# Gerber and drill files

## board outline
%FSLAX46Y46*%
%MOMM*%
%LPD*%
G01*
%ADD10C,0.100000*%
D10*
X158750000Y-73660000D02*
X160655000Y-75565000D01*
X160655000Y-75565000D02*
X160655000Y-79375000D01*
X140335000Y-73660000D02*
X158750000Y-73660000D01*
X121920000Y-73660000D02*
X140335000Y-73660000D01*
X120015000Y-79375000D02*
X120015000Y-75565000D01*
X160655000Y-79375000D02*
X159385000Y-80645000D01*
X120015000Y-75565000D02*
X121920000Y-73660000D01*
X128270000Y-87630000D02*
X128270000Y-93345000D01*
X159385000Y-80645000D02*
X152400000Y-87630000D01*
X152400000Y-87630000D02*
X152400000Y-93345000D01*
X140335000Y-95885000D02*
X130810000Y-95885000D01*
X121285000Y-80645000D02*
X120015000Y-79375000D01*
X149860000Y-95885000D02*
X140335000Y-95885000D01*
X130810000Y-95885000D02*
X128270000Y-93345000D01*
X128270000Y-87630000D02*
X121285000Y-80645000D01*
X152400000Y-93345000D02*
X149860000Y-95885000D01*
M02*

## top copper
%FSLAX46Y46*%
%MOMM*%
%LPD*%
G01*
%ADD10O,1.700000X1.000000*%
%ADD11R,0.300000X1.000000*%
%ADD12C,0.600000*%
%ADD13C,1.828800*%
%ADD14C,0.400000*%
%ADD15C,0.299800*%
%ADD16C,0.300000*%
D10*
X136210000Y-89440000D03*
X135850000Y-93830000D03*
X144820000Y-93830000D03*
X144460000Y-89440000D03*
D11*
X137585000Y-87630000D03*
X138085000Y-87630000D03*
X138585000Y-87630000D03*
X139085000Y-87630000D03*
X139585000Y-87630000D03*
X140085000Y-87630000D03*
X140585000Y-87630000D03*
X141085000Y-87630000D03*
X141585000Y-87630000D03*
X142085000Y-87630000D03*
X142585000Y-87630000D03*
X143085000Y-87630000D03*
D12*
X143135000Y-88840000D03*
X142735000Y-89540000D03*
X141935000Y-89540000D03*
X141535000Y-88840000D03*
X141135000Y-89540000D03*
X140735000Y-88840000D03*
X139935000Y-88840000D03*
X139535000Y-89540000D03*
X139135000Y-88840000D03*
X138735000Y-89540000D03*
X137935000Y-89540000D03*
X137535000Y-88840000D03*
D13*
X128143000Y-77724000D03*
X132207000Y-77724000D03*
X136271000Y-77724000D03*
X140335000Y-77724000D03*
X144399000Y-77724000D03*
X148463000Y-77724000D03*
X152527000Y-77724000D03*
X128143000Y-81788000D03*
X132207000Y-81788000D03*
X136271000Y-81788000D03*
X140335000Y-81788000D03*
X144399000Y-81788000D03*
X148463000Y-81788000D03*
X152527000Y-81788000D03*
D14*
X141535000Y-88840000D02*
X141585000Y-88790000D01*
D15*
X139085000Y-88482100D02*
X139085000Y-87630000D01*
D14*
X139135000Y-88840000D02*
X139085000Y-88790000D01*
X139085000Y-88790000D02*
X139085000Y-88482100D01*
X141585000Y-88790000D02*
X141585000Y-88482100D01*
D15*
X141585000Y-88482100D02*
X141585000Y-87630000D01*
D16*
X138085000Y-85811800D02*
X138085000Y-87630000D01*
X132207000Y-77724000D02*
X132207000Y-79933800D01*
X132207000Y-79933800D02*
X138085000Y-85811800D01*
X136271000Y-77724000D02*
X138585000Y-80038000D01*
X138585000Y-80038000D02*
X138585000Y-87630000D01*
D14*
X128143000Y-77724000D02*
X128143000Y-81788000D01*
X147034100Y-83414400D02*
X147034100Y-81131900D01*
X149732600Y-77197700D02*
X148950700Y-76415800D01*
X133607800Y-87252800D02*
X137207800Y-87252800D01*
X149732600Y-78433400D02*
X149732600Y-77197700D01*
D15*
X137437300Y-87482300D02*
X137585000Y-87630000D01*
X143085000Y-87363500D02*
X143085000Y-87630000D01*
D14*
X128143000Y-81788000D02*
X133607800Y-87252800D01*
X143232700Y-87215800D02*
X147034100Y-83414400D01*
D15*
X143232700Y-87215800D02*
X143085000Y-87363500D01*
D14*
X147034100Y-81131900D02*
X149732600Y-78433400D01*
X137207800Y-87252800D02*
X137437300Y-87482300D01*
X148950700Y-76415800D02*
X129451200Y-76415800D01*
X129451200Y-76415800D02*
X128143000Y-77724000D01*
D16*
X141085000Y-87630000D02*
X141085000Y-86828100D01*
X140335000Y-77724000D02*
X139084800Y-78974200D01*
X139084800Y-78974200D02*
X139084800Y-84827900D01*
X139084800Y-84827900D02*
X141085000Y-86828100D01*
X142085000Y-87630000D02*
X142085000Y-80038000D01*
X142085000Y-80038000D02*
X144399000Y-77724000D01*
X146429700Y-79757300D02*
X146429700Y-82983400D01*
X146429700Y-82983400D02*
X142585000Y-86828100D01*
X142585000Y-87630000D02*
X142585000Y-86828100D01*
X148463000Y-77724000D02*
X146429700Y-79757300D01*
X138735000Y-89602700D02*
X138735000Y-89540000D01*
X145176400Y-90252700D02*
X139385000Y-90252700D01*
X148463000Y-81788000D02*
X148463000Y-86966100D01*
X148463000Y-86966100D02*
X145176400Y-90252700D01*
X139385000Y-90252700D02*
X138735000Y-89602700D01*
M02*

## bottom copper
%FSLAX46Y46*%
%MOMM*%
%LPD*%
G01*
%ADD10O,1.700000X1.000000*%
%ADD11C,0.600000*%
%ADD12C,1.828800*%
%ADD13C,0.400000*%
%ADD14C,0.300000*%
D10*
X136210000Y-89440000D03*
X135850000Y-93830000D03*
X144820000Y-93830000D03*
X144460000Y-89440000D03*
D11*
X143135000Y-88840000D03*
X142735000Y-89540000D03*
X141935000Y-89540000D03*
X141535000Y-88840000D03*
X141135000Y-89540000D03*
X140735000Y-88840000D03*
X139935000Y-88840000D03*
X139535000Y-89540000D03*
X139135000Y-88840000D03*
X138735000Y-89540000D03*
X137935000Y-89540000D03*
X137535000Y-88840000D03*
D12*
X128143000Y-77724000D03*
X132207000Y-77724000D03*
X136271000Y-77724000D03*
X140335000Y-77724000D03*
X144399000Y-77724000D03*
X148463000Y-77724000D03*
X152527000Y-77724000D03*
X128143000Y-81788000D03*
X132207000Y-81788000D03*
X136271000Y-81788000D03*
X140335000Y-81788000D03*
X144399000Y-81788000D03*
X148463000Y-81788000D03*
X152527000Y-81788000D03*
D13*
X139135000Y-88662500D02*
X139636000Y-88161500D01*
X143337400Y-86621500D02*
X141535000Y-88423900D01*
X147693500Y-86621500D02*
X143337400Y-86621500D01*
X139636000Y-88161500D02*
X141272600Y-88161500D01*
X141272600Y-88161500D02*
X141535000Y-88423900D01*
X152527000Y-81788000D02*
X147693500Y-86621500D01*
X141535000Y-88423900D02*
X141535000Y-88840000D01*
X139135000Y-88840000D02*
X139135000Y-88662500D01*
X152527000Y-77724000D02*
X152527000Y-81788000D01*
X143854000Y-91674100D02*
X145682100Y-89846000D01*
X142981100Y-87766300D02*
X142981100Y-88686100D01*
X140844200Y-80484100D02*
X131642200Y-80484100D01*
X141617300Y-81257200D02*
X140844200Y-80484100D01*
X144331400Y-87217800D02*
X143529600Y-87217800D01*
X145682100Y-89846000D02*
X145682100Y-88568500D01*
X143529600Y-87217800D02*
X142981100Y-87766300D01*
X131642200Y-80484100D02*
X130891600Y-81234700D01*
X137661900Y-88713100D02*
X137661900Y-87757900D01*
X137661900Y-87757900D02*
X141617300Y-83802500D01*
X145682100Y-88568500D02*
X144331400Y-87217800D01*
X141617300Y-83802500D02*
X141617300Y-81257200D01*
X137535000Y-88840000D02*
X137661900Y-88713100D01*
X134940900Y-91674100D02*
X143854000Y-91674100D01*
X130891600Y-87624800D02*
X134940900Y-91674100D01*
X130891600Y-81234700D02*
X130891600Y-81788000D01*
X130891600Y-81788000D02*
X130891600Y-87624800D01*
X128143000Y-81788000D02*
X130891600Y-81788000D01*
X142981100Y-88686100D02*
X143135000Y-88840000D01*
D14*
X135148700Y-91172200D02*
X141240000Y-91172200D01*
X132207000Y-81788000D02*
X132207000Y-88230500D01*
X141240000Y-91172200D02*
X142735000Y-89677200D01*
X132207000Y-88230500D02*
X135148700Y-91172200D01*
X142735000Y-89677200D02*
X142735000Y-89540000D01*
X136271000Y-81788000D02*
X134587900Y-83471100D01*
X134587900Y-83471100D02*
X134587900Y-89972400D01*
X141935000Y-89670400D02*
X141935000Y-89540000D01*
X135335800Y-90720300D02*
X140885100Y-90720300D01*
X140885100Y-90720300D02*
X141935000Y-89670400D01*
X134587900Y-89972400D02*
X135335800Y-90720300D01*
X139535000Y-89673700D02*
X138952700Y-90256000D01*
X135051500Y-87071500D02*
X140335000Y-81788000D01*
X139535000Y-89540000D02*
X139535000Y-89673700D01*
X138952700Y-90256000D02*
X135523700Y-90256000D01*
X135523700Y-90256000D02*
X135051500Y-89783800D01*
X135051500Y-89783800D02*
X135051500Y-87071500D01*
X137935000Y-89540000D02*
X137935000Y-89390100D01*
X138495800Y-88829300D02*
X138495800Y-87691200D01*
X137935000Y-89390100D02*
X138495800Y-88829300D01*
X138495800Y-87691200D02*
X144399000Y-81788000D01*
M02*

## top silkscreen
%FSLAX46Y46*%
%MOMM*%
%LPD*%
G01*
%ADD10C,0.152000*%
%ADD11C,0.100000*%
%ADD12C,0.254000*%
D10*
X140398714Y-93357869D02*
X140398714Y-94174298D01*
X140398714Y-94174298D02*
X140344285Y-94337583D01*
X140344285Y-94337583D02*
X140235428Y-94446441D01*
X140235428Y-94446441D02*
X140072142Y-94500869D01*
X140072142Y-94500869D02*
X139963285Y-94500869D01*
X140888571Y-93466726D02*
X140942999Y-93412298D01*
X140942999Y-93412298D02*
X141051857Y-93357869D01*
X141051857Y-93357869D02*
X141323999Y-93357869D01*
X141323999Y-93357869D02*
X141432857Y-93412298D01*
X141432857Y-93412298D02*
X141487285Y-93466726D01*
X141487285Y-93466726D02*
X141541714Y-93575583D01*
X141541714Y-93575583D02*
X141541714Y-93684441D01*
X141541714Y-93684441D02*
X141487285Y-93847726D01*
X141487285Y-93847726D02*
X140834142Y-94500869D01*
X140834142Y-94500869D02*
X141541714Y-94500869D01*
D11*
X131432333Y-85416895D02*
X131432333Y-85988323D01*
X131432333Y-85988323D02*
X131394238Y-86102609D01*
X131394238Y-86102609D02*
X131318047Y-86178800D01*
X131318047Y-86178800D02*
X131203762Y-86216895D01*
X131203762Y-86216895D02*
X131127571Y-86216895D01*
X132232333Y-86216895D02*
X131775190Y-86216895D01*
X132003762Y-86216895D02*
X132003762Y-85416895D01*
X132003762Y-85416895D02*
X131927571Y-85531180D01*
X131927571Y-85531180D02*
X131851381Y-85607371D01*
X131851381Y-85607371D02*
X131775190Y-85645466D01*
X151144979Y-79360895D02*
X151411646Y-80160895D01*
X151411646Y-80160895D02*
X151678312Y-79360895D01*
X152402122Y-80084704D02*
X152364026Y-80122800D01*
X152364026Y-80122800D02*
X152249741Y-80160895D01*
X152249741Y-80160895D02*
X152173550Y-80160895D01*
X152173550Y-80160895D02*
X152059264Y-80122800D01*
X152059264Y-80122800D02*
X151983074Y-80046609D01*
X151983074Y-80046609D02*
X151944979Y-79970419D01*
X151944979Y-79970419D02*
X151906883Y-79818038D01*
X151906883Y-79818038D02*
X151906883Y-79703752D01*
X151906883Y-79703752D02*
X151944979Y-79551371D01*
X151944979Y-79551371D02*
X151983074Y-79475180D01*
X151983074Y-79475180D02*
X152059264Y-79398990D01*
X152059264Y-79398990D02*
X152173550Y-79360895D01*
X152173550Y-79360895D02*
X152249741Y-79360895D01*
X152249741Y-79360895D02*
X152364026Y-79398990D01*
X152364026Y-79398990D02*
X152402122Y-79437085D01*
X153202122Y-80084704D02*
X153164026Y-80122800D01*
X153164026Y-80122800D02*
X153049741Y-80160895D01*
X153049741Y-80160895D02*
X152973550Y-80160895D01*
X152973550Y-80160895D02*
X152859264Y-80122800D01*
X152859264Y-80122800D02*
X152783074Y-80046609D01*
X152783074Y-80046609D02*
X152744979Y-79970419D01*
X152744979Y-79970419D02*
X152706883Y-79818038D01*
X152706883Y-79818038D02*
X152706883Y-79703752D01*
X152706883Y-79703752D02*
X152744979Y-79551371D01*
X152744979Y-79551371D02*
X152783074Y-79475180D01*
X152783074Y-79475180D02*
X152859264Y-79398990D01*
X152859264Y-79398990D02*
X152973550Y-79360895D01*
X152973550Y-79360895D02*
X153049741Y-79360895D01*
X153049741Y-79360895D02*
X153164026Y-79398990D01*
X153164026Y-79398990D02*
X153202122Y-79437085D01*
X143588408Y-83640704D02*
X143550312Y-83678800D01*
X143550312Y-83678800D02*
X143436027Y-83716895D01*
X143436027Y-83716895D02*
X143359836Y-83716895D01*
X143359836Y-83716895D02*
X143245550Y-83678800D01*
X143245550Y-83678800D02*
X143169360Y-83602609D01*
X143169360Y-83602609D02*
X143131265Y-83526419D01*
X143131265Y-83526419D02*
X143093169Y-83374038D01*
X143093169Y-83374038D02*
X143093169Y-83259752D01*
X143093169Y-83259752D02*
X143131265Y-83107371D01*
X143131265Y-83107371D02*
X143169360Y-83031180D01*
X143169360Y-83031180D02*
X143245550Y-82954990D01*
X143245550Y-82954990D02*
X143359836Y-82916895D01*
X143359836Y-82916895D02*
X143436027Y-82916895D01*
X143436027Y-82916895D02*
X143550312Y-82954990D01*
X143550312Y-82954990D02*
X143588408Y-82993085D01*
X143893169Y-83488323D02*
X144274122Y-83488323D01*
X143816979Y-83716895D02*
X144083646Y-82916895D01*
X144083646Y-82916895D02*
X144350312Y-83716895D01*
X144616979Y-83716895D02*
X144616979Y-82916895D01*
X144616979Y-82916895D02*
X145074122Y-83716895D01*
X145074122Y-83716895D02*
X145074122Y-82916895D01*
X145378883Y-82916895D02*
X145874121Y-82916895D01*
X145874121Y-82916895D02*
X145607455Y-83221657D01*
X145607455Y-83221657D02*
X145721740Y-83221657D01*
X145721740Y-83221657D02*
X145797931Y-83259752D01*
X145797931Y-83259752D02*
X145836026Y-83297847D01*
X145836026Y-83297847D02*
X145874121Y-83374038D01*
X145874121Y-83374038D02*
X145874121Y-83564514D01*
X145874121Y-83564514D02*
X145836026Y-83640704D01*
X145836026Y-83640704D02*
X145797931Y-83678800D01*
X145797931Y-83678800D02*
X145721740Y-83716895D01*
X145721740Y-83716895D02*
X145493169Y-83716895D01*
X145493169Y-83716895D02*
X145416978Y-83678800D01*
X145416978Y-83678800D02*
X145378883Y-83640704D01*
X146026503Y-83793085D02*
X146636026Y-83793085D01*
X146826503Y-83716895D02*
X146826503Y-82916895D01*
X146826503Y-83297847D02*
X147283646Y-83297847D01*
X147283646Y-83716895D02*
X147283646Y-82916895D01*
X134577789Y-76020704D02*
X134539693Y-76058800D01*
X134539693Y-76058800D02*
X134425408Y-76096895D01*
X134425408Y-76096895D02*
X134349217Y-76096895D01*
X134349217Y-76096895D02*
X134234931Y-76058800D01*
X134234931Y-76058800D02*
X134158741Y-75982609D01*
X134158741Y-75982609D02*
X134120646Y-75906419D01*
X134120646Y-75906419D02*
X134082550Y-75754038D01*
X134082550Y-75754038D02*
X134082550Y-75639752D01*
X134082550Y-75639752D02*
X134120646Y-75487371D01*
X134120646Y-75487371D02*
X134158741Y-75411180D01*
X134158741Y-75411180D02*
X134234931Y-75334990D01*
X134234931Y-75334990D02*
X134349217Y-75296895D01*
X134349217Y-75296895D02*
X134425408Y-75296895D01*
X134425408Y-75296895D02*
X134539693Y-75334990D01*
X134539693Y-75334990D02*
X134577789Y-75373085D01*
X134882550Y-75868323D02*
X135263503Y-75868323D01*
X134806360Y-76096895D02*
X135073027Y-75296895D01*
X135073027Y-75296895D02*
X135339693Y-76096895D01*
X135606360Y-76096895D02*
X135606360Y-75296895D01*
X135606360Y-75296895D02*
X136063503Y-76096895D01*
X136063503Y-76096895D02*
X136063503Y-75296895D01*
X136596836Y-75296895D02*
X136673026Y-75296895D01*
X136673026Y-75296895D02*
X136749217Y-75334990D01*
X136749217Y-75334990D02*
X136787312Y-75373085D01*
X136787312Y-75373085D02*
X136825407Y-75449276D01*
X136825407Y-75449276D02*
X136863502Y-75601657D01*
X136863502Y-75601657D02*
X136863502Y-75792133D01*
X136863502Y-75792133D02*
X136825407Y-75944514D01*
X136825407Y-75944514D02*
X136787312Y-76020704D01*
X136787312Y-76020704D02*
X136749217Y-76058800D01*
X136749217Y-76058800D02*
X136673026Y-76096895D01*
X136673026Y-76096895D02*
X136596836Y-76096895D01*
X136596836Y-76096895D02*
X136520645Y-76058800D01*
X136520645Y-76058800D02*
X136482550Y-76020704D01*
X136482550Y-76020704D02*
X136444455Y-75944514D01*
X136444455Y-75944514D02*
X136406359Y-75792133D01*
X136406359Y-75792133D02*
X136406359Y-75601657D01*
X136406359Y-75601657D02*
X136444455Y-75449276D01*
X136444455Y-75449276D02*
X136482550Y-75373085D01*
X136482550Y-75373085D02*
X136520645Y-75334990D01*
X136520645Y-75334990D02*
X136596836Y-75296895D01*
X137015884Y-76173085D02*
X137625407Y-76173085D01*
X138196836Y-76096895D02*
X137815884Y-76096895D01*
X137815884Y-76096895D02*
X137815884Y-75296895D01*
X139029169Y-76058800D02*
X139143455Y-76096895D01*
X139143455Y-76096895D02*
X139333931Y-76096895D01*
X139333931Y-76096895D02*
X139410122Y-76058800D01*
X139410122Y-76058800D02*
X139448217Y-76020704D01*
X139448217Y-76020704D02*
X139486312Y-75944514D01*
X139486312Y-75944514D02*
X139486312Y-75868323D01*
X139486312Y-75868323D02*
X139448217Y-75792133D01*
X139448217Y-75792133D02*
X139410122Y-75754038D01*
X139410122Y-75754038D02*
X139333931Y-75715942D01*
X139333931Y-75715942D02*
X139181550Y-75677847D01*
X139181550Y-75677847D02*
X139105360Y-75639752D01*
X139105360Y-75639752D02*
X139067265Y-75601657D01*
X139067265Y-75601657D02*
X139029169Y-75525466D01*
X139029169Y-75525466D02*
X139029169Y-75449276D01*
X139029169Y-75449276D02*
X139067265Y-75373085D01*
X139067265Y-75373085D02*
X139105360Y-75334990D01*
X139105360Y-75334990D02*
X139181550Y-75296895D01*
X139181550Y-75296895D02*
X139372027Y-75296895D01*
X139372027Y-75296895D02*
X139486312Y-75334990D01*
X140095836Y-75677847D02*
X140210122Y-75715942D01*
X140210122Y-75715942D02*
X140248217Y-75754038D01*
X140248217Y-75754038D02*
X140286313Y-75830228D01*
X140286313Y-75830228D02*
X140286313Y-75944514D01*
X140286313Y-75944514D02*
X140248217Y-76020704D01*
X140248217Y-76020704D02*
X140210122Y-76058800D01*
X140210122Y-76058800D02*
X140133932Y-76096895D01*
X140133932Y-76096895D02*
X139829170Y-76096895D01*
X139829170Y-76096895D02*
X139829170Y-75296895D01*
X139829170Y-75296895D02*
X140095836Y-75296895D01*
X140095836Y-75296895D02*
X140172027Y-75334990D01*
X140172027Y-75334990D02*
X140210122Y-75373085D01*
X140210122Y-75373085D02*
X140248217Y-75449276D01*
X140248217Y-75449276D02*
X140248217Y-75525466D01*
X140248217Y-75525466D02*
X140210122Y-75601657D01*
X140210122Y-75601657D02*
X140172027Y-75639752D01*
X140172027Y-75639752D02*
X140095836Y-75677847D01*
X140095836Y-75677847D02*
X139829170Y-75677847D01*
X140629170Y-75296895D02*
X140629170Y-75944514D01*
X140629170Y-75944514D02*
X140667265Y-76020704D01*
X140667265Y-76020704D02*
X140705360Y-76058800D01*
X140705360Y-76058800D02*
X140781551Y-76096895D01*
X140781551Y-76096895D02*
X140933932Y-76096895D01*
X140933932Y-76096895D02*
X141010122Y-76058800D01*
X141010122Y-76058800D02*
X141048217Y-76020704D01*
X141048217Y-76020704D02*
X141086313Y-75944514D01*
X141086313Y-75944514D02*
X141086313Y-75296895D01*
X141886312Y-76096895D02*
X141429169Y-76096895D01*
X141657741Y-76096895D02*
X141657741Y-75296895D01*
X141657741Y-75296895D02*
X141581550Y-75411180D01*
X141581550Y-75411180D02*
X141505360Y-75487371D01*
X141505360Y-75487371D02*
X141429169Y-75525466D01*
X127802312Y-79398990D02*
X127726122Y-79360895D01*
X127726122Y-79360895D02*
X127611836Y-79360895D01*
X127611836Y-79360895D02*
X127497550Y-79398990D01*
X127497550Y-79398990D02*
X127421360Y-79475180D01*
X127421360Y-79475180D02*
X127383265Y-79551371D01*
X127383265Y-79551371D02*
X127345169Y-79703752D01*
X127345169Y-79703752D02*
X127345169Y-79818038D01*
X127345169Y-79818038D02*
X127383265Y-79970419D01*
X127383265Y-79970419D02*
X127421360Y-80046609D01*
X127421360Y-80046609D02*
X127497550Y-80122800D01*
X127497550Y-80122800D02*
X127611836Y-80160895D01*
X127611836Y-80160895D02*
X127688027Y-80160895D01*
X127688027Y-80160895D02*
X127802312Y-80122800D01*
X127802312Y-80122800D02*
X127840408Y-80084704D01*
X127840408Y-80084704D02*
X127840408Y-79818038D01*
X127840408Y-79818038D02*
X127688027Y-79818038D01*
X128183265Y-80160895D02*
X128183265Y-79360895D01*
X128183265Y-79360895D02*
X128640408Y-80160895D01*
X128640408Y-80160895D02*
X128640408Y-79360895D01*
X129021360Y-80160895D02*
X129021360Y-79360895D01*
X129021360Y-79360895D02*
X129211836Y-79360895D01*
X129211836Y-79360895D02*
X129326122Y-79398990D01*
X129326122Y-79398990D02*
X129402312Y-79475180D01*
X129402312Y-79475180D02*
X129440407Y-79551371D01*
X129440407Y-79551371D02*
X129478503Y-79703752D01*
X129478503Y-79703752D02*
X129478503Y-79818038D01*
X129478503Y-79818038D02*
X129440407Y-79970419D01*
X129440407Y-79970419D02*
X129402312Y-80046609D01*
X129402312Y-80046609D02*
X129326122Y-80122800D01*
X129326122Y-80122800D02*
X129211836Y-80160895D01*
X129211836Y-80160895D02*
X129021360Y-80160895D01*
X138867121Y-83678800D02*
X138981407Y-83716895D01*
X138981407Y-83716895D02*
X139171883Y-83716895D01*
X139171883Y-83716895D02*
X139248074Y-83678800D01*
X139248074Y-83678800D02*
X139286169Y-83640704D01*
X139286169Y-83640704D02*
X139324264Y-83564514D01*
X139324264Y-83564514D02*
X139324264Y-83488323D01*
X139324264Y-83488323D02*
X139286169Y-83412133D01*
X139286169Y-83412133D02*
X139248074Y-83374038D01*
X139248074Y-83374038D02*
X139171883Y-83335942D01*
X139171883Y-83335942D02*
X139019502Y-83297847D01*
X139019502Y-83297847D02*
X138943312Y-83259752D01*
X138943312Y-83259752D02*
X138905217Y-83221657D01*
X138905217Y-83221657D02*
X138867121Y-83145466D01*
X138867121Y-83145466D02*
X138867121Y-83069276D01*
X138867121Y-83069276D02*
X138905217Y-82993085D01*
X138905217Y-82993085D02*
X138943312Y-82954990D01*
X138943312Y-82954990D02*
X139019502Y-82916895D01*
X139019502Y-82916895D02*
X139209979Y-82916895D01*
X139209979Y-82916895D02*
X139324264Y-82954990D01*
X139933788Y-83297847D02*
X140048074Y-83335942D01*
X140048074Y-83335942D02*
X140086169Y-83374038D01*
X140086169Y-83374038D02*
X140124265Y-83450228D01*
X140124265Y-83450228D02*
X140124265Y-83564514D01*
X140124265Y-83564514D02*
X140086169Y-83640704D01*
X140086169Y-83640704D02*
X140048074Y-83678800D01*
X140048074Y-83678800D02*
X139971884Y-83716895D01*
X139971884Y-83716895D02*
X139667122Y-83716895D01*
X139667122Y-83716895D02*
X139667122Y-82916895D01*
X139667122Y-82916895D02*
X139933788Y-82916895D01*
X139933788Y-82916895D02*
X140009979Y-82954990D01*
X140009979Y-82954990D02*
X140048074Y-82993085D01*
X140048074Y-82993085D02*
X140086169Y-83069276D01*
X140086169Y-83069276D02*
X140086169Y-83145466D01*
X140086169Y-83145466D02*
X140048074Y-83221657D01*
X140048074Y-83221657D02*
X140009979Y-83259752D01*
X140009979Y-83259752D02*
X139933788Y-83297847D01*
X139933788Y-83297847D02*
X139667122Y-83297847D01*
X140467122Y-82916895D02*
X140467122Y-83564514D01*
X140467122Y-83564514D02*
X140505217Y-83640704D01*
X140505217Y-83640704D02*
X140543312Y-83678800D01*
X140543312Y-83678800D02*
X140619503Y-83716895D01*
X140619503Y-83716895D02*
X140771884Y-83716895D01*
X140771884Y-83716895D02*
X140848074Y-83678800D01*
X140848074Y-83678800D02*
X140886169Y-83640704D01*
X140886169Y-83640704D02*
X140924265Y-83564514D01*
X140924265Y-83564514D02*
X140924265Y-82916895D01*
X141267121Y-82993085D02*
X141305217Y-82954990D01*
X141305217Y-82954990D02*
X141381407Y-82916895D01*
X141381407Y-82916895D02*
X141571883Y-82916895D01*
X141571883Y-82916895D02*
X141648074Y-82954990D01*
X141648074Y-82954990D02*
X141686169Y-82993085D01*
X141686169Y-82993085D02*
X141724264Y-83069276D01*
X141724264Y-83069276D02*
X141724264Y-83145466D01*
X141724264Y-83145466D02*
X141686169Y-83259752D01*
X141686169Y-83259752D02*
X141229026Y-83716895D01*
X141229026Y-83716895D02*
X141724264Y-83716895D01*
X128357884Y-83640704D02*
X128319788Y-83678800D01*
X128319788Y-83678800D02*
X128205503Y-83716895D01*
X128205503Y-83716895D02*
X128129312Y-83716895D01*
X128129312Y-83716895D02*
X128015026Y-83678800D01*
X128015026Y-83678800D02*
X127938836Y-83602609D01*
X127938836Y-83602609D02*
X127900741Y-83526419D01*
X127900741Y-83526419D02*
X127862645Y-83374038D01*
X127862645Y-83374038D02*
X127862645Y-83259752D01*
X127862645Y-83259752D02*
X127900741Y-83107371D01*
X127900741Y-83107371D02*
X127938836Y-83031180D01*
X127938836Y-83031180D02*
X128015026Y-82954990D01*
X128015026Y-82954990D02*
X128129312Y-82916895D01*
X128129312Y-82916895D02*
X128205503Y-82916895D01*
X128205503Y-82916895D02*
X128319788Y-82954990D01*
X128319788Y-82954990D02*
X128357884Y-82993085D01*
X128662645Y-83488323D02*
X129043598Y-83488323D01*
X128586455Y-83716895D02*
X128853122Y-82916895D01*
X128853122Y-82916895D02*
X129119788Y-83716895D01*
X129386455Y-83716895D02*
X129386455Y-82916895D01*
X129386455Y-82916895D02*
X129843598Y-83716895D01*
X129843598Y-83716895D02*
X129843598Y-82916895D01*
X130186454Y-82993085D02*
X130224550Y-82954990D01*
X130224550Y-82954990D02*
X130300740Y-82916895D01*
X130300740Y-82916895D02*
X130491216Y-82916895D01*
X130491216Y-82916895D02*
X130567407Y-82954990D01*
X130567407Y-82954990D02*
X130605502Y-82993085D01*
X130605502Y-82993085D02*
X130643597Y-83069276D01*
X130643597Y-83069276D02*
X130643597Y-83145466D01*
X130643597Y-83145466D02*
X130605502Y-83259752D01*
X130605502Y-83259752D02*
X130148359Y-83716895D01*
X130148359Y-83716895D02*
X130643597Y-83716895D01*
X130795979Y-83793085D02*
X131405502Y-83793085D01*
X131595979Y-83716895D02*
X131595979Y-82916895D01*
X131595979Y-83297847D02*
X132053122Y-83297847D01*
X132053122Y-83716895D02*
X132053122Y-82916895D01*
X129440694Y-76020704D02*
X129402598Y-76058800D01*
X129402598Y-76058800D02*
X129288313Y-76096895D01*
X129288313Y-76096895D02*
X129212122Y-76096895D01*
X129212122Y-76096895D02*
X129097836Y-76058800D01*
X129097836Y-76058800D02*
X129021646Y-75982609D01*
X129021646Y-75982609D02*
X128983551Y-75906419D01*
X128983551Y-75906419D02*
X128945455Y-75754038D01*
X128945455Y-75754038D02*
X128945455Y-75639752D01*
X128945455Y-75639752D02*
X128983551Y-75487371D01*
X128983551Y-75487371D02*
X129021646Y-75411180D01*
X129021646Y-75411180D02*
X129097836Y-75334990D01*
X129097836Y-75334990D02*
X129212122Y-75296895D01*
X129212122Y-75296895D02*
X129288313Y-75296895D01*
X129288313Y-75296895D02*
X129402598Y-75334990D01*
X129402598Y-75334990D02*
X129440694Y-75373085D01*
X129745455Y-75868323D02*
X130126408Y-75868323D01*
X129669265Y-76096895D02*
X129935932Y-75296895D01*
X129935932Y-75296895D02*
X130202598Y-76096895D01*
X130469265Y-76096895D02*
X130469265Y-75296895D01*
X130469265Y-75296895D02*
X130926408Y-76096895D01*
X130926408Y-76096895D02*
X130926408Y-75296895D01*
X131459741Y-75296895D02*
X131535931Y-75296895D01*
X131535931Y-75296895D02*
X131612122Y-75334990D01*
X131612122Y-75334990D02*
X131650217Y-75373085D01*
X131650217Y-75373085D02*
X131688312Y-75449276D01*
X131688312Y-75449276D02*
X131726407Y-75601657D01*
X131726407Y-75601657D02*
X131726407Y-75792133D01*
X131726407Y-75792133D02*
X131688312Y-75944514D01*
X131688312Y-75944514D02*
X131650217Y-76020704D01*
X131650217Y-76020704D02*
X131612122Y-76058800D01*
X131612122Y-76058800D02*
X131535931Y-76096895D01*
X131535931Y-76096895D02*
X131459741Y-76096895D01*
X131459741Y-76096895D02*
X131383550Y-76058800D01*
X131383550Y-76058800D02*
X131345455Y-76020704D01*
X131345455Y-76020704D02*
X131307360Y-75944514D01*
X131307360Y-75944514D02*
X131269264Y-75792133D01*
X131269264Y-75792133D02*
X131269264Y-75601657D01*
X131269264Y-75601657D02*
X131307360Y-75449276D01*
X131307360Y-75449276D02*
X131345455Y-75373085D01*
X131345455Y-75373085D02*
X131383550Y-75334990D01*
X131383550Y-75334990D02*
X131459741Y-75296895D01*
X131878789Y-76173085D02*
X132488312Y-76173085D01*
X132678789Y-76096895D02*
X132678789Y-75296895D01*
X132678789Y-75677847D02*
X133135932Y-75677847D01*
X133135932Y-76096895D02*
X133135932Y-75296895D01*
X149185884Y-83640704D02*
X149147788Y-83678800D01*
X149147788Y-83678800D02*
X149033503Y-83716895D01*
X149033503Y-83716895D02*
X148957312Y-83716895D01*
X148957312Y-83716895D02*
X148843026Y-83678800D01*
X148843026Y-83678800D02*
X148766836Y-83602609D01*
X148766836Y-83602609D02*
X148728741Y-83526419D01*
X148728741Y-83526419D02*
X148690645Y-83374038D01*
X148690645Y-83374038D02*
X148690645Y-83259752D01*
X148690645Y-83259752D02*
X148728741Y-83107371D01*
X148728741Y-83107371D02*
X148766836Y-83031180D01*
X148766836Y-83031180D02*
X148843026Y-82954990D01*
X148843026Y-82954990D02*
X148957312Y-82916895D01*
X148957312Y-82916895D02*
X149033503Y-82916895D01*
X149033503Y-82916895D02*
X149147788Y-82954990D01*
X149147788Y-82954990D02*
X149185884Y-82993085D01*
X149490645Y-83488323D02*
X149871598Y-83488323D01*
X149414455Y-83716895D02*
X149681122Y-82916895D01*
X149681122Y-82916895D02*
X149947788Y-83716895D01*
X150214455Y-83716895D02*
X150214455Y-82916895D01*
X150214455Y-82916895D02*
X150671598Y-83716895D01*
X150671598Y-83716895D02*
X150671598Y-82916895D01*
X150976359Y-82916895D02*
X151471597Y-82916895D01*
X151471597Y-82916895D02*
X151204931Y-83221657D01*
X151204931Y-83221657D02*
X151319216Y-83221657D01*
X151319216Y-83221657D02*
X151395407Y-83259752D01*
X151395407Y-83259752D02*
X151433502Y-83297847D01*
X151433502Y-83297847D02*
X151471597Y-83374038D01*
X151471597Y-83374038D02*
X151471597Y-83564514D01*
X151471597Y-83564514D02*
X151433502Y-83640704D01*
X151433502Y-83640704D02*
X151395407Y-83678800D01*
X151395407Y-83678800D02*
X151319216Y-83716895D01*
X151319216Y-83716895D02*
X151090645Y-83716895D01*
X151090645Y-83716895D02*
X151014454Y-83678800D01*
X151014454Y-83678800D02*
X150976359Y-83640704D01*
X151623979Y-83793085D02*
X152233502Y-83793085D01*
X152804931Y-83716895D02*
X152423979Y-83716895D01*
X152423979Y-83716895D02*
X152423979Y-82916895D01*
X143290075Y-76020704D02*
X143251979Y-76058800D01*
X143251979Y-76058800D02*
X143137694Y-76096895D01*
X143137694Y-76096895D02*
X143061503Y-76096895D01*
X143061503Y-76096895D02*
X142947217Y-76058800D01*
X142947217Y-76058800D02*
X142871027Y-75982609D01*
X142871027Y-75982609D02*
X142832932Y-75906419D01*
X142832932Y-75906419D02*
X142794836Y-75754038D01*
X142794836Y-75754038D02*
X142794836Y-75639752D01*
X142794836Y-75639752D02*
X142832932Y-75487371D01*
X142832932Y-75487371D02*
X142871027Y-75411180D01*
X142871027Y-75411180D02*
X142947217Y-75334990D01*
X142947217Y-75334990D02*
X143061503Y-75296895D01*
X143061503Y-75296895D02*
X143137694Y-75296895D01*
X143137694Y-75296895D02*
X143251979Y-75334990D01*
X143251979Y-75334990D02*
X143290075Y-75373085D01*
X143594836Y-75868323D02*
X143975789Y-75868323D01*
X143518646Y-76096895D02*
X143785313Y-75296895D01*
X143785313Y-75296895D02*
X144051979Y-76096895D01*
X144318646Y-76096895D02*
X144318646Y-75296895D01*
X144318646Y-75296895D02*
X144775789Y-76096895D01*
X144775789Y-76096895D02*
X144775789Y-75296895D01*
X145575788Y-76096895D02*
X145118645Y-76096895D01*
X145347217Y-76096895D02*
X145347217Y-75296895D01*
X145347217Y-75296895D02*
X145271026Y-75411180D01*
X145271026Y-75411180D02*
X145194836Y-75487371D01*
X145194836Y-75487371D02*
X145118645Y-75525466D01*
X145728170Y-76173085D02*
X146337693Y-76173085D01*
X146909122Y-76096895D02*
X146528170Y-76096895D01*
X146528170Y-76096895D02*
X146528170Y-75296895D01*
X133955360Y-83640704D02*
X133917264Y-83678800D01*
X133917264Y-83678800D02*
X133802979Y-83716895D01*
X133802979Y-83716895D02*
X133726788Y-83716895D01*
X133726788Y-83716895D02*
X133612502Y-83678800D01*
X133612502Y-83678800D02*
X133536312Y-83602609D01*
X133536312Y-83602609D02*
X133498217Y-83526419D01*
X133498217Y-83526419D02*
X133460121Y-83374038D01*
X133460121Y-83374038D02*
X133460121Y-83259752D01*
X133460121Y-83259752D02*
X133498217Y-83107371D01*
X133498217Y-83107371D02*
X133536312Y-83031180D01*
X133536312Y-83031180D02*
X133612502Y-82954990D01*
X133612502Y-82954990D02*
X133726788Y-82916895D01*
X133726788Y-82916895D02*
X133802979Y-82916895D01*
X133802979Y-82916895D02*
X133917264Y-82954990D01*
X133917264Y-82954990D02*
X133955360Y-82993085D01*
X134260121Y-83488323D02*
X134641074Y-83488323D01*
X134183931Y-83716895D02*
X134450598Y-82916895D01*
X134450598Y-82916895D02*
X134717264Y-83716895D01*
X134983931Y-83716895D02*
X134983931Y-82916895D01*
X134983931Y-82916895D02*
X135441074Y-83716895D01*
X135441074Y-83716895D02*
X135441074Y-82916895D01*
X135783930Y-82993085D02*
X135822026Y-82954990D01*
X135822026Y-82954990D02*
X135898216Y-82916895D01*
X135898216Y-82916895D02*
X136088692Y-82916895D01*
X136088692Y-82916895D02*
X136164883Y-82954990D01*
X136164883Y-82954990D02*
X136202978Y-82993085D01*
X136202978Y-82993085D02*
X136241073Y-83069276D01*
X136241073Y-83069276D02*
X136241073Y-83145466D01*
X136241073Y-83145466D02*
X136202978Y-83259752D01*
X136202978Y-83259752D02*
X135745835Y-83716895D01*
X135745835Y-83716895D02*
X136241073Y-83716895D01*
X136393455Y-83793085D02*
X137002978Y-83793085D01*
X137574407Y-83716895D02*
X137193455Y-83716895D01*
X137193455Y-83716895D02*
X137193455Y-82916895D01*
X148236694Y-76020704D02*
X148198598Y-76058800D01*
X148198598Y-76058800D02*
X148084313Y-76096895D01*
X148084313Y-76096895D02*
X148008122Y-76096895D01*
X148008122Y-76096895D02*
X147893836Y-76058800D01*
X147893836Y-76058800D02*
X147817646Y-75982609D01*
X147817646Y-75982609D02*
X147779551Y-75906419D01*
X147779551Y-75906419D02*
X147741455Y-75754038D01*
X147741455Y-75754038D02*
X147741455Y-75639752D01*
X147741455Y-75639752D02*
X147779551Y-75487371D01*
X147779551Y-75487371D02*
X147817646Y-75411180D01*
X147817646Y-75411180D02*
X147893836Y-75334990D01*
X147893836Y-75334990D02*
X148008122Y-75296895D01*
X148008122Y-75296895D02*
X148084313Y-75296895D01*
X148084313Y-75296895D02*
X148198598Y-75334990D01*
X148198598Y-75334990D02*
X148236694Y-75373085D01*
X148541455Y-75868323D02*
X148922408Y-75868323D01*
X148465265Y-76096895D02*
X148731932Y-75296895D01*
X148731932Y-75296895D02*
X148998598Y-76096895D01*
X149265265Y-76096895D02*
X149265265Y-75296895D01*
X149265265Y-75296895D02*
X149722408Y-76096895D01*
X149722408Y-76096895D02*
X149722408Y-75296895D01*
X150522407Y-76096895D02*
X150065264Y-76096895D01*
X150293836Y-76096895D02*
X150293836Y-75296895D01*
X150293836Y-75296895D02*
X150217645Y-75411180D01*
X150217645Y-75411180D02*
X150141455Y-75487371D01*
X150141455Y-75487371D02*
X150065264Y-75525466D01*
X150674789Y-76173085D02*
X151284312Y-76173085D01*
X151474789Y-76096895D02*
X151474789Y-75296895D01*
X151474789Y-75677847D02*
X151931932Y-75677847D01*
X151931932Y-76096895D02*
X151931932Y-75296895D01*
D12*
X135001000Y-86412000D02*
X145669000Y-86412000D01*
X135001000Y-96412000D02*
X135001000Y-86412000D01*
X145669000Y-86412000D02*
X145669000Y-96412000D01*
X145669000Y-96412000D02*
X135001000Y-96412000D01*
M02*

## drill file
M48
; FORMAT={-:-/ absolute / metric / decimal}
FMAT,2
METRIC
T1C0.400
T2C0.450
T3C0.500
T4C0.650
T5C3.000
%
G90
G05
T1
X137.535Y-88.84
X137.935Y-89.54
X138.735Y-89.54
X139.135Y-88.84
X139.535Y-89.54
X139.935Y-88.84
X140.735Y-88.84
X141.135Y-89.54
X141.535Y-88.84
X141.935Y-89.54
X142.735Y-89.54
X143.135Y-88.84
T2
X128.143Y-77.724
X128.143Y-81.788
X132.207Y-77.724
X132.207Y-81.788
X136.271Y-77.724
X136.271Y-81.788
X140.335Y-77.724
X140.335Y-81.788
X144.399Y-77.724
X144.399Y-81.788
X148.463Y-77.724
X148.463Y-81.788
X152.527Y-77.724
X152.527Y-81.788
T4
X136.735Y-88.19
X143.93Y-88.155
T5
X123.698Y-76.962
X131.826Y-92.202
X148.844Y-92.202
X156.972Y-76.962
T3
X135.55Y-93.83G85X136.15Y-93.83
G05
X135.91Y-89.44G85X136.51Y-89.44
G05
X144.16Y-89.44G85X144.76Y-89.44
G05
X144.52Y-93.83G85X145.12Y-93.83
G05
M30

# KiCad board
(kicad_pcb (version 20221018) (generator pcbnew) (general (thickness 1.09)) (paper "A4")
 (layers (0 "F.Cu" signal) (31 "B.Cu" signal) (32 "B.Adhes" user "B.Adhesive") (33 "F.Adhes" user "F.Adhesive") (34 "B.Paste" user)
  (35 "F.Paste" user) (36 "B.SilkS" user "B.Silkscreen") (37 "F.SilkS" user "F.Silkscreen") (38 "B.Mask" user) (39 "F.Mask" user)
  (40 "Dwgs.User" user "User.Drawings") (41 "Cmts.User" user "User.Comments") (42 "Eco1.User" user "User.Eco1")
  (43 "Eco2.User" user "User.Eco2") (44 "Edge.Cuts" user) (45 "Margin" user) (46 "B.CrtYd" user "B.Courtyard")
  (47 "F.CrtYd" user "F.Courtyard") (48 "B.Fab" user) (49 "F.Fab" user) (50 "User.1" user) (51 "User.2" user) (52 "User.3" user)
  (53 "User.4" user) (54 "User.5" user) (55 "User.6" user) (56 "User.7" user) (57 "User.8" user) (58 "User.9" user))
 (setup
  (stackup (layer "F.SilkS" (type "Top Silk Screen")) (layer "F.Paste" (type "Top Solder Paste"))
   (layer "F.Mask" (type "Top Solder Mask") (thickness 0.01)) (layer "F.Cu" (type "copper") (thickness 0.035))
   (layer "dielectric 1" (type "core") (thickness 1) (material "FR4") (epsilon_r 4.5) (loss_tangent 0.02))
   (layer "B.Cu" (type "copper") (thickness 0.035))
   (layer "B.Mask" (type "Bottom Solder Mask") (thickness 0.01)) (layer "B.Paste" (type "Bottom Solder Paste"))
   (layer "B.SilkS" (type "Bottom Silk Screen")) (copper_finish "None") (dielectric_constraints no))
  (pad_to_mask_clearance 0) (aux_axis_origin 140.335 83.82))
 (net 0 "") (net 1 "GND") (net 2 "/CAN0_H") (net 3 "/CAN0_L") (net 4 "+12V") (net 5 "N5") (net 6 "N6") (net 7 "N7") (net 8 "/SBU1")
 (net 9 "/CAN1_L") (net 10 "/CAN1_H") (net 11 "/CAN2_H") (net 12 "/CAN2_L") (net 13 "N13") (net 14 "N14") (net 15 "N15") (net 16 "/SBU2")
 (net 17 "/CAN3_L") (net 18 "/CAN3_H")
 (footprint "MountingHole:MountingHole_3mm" (layer "F.Cu") (at 123.698 76.962)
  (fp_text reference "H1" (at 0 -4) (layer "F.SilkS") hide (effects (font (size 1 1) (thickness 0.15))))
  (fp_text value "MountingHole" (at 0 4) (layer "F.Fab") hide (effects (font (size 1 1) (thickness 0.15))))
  (pad "" np_thru_hole circle (at 0 0) (size 3 3) (drill 3) (layers "*.Cu" "*.Mask")))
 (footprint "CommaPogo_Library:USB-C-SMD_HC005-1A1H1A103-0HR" (layer "F.Cu") (at 140.335 90.73)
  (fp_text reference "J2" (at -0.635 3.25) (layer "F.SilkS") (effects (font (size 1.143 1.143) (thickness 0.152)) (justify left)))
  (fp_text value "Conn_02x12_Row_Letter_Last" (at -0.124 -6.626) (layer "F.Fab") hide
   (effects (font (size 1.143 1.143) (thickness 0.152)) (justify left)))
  (fp_line (start -5.334 -4.318) (end 5.334 -4.318) (stroke (width 0.254) (type solid)) (layer "F.SilkS"))
  (fp_line (start -5.334 5.682) (end -5.334 -4.318) (stroke (width 0.254) (type solid)) (layer "F.SilkS"))
  (fp_line (start 5.334 -4.318) (end 5.334 5.682) (stroke (width 0.254) (type solid)) (layer "F.SilkS"))
  (fp_line (start 5.334 5.682) (end -5.334 5.682) (stroke (width 0.254) (type solid)) (layer "F.SilkS"))
  (pad "" np_thru_hole circle (at -3.6 -2.54) (size 0.65 0.65) (drill 0.65) (layers "*.Cu" "*.Mask"))
  (pad "" np_thru_hole circle (at 3.595 -2.575) (size 0.65 0.65) (drill 0.65) (layers "*.Cu" "*.Mask"))
  (pad "1" thru_hole oval (at -4.125 -1.29 90) (size 1 1.7) (drill oval 0.5 1.1) (layers "*.Cu" "*.Paste" "*.Mask"))
  (pad "2" thru_hole oval (at -4.485 3.1 90) (size 1 1.7) (drill oval 0.5 1.1) (layers "*.Cu" "*.Paste" "*.Mask"))
  (pad "3" thru_hole oval (at 4.485 3.1 90) (size 1 1.7) (drill oval 0.5 1.1) (layers "*.Cu" "*.Paste" "*.Mask"))
  (pad "4" thru_hole oval (at 4.125 -1.29 90) (size 1 1.7) (drill oval 0.5 1.1) (layers "*.Cu" "*.Paste" "*.Mask"))
  (pad "A1" smd rect (at -2.75 -3.1) (size 0.3 1) (layers "F.Cu" "F.Paste" "F.Mask") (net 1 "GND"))
  (pad "A2" smd rect (at -2.25 -3.1) (size 0.3 1) (layers "F.Cu" "F.Paste" "F.Mask") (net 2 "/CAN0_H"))
  (pad "A3" smd rect (at -1.75 -3.1) (size 0.3 1) (layers "F.Cu" "F.Paste" "F.Mask") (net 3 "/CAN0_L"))
  (pad "A4" smd rect (at -1.25 -3.1) (size 0.3 1) (layers "F.Cu" "F.Paste" "F.Mask") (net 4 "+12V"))
  (pad "A5" smd rect (at -0.75 -3.1) (size 0.3 1) (layers "F.Cu" "F.Paste" "F.Mask") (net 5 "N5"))
  (pad "A6" smd rect (at -0.25 -3.1) (size 0.3 1) (layers "F.Cu" "F.Paste" "F.Mask") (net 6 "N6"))
  (pad "A7" smd rect (at 0.25 -3.1) (size 0.3 1) (layers "F.Cu" "F.Paste" "F.Mask") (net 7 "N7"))
  (pad "A8" smd rect (at 0.75 -3.1) (size 0.3 1) (layers "F.Cu" "F.Paste" "F.Mask") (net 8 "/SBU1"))
  (pad "A9" smd rect (at 1.25 -3.1) (size 0.3 1) (layers "F.Cu" "F.Paste" "F.Mask") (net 4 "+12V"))
  (pad "A10" smd rect (at 1.75 -3.1) (size 0.3 1) (layers "F.Cu" "F.Paste" "F.Mask") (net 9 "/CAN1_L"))
  (pad "A11" smd rect (at 2.25 -3.1) (size 0.3 1) (layers "F.Cu" "F.Paste" "F.Mask") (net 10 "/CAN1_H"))
  (pad "A12" smd rect (at 2.75 -3.1) (size 0.3 1) (layers "F.Cu" "F.Paste" "F.Mask") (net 1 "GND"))
  (pad "B1" thru_hole circle (at 2.8 -1.89) (size 0.6 0.6) (drill 0.4) (layers "*.Cu" "*.Paste" "*.Mask") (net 1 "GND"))
  (pad "B2" thru_hole circle (at 2.4 -1.19) (size 0.6 0.6) (drill 0.4) (layers "*.Cu" "*.Paste" "*.Mask") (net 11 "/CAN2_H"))
  (pad "B3" thru_hole circle (at 1.6 -1.19) (size 0.6 0.6) (drill 0.4) (layers "*.Cu" "*.Paste" "*.Mask") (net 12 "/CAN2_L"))
  (pad "B4" thru_hole circle (at 1.2 -1.89) (size 0.6 0.6) (drill 0.4) (layers "*.Cu" "*.Paste" "*.Mask") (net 4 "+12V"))
  (pad "B5" thru_hole circle (at 0.8 -1.19) (size 0.6 0.6) (drill 0.4) (layers "*.Cu" "*.Paste" "*.Mask") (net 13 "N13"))
  (pad "B6" thru_hole circle (at 0.4 -1.89) (size 0.6 0.6) (drill 0.4) (layers "*.Cu" "*.Paste" "*.Mask") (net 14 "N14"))
  (pad "B7" thru_hole circle (at -0.4 -1.89) (size 0.6 0.6) (drill 0.4) (layers "*.Cu" "*.Paste" "*.Mask") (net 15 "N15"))
  (pad "B8" thru_hole circle (at -0.8 -1.19) (size 0.6 0.6) (drill 0.4) (layers "*.Cu" "*.Paste" "*.Mask") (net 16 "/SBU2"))
  (pad "B9" thru_hole circle (at -1.2 -1.89) (size 0.6 0.6) (drill 0.4) (layers "*.Cu" "*.Paste" "*.Mask") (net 4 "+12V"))
  (pad "B10" thru_hole circle (at -1.6 -1.19) (size 0.6 0.6) (drill 0.4) (layers "*.Cu" "*.Paste" "*.Mask") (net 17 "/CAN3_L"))
  (pad "B11" thru_hole circle (at -2.4 -1.19) (size 0.6 0.6) (drill 0.4) (layers "*.Cu" "*.Paste" "*.Mask") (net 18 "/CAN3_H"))
  (pad "B12" thru_hole circle (at -2.8 -1.89) (size 0.6 0.6) (drill 0.4) (layers "*.Cu" "*.Paste" "*.Mask") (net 1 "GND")))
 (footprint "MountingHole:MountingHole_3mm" (layer "F.Cu") (at 148.844 92.202)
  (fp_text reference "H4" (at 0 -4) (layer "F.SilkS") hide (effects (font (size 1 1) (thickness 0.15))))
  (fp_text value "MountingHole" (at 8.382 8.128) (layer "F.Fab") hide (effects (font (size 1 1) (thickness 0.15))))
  (pad "" np_thru_hole circle (at 0 0) (size 3 3) (drill 3) (layers "*.Cu" "*.Mask")))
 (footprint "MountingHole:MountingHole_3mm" (layer "F.Cu") (at 131.826 92.202)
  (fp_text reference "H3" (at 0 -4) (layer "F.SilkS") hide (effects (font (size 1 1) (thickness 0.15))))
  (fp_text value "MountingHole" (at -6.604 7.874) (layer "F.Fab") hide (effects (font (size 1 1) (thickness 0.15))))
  (pad "" np_thru_hole circle (at 0 0) (size 3 3) (drill 3) (layers "*.Cu" "*.Mask")))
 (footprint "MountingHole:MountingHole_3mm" (layer "F.Cu") (at 156.972 76.962)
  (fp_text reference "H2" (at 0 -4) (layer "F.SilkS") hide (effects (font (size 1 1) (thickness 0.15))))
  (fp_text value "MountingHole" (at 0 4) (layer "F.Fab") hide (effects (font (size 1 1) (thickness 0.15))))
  (pad "" np_thru_hole circle (at 0 0) (size 3 3) (drill 3) (layers "*.Cu" "*.Mask")))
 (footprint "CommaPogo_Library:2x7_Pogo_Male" (layer "F.Cu") (at 140.335 83.82)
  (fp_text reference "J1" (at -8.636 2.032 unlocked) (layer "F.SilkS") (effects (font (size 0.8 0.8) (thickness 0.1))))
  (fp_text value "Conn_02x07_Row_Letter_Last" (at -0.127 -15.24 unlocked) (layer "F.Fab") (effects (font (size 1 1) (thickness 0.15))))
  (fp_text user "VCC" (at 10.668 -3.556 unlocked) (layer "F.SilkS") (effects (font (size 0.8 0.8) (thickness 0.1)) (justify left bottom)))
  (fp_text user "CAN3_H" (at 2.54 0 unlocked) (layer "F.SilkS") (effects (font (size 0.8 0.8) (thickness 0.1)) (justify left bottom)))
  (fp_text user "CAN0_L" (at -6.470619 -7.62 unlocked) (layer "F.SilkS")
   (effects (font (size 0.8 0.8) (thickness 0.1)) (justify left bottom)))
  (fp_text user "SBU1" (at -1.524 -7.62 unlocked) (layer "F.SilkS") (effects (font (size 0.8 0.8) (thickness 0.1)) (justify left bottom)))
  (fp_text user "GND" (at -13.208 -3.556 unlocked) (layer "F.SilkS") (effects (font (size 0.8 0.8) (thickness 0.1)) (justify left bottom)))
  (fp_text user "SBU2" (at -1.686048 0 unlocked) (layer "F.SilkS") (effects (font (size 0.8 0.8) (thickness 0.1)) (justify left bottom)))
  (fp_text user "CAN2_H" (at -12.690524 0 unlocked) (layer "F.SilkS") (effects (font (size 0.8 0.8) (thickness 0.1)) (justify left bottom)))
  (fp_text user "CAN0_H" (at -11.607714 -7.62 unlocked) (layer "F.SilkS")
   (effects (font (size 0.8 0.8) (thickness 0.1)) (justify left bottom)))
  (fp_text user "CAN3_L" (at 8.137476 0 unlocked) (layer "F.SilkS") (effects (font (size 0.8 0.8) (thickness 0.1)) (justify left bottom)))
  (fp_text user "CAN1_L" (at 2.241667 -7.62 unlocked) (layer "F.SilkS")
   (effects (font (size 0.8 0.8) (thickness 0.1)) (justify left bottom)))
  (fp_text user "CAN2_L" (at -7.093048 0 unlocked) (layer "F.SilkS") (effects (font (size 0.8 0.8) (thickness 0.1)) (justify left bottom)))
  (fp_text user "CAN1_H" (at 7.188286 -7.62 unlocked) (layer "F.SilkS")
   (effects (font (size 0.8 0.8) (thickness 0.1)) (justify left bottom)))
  (pad "1" thru_hole circle (at -12.192 -6.096) (size 1.8288 1.8288) (drill 0.45) (layers "*.Cu" "*.Mask") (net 1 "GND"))
  (pad "2" thru_hole circle (at -8.128 -6.096) (size 1.8288 1.8288) (drill 0.45) (layers "*.Cu" "*.Mask") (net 2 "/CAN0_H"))
  (pad "3" thru_hole circle (at -4.064 -6.096) (size 1.8288 1.8288) (drill 0.45) (layers "*.Cu" "*.Mask") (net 3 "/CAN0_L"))
  (pad "4" thru_hole circle (at 0 -6.096) (size 1.8288 1.8288) (drill 0.45) (layers "*.Cu" "*.Mask") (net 8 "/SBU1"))
  (pad "5" thru_hole circle (at 4.064 -6.096) (size 1.8288 1.8288) (drill 0.45) (layers "*.Cu" "*.Mask") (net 9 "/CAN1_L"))
  (pad "6" thru_hole circle (at 8.128 -6.096) (size 1.8288 1.8288) (drill 0.45) (layers "*.Cu" "*.Mask") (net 10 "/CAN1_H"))
  (pad "7" thru_hole circle (at 12.192 -6.096) (size 1.8288 1.8288) (drill 0.45) (layers "*.Cu" "*.Mask") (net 4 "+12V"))
  (pad "8" thru_hole circle (at -12.192 -2.032) (size 1.8288 1.8288) (drill 0.45) (layers "*.Cu" "*.Mask") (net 1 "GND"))
  (pad "9" thru_hole circle (at -8.128 -2.032) (size 1.8288 1.8288) (drill 0.45) (layers "*.Cu" "*.Mask") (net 11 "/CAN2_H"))
  (pad "10" thru_hole circle (at -4.064 -2.032) (size 1.8288 1.8288) (drill 0.45) (layers "*.Cu" "*.Mask") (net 12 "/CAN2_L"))
  (pad "11" thru_hole circle (at 0 -2.032) (size 1.8288 1.8288) (drill 0.45) (layers "*.Cu" "*.Mask") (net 16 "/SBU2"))
  (pad "12" thru_hole circle (at 4.064 -2.032) (size 1.8288 1.8288) (drill 0.45) (layers "*.Cu" "*.Mask") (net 18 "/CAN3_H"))
  (pad "13" thru_hole circle (at 8.128 -2.032) (size 1.8288 1.8288) (drill 0.45) (layers "*.Cu" "*.Mask") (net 17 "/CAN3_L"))
  (pad "14" thru_hole circle (at 12.192 -2.032) (size 1.8288 1.8288) (drill 0.45) (layers "*.Cu" "*.Mask") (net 4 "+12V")))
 (gr_line (start 158.75 73.66) (end 160.655 75.565) (stroke (width 0.1) (type default)) (layer "Edge.Cuts"))
 (gr_line (start 160.655 75.565) (end 160.655 79.375) (stroke (width 0.1) (type default)) (layer "Edge.Cuts"))
 (gr_line (start 140.335 73.66) (end 158.75 73.66) (stroke (width 0.1) (type default)) (layer "Edge.Cuts"))
 (gr_line (start 121.92 73.66) (end 140.335 73.66) (stroke (width 0.1) (type default)) (layer "Edge.Cuts"))
 (gr_line (start 120.015 79.375) (end 120.015 75.565) (stroke (width 0.1) (type default)) (layer "Edge.Cuts"))
 (gr_line (start 160.655 79.375) (end 159.385 80.645) (stroke (width 0.1) (type default)) (layer "Edge.Cuts"))
 (gr_line (start 120.015 75.565) (end 121.92 73.66) (stroke (width 0.1) (type default)) (layer "Edge.Cuts"))
 (gr_line (start 128.27 87.63) (end 128.27 93.345) (stroke (width 0.1) (type default)) (layer "Edge.Cuts"))
 (gr_line (start 159.385 80.645) (end 152.4 87.63) (stroke (width 0.1) (type default)) (layer "Edge.Cuts"))
 (gr_line (start 152.4 87.63) (end 152.4 93.345) (stroke (width 0.1) (type default)) (layer "Edge.Cuts"))
 (gr_line (start 140.335 95.885) (end 130.81 95.885) (stroke (width 0.1) (type default)) (layer "Edge.Cuts"))
 (gr_line (start 121.285 80.645) (end 120.015 79.375) (stroke (width 0.1) (type default)) (layer "Edge.Cuts"))
 (gr_line (start 149.86 95.885) (end 140.335 95.885) (stroke (width 0.1) (type default)) (layer "Edge.Cuts"))
 (gr_line (start 130.81 95.885) (end 128.27 93.345) (stroke (width 0.1) (type default)) (layer "Edge.Cuts"))
 (gr_line (start 128.27 87.63) (end 121.285 80.645) (stroke (width 0.1) (type default)) (layer "Edge.Cuts"))
 (gr_line (start 152.4 93.345) (end 149.86 95.885) (stroke (width 0.1) (type default)) (layer "Edge.Cuts"))
 (segment (start 141.535 88.84) (end 141.585 88.79) (width 0.4) (layer "F.Cu") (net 4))
 (segment (start 139.085 88.4821) (end 139.085 87.63) (width 0.2998) (layer "F.Cu") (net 4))
 (segment (start 139.135 88.84) (end 139.085 88.79) (width 0.4) (layer "F.Cu") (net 4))
 (segment (start 139.085 88.79) (end 139.085 88.4821) (width 0.4) (layer "F.Cu") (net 4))
 (segment (start 141.585 88.79) (end 141.585 88.4821) (width 0.4) (layer "F.Cu") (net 4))
 (segment (start 141.585 88.4821) (end 141.585 87.63) (width 0.2998) (layer "F.Cu") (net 4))
 (segment (start 139.135 88.6625) (end 139.636 88.1615) (width 0.4) (layer "B.Cu") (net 4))
 (segment (start 143.3374 86.6215) (end 141.535 88.4239) (width 0.4) (layer "B.Cu") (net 4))
 (segment (start 147.6935 86.6215) (end 143.3374 86.6215) (width 0.4) (layer "B.Cu") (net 4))
 (segment (start 139.636 88.1615) (end 141.2726 88.1615) (width 0.4) (layer "B.Cu") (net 4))
 (segment (start 141.2726 88.1615) (end 141.535 88.4239) (width 0.4) (layer "B.Cu") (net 4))
 (segment (start 152.527 81.788) (end 147.6935 86.6215) (width 0.4) (layer "B.Cu") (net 4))
 (segment (start 141.535 88.4239) (end 141.535 88.84) (width 0.4) (layer "B.Cu") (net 4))
 (segment (start 139.135 88.84) (end 139.135 88.6625) (width 0.4) (layer "B.Cu") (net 4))
 (segment (start 152.527 77.724) (end 152.527 81.788) (width 0.4) (layer "B.Cu") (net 4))
 (segment (start 138.085 85.8118) (end 138.085 87.63) (width 0.3) (layer "F.Cu") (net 2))
 (segment (start 132.207 77.724) (end 132.207 79.9338) (width 0.3) (layer "F.Cu") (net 2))
 (segment (start 132.207 79.9338) (end 138.085 85.8118) (width 0.3) (layer "F.Cu") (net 2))
 (segment (start 136.271 77.724) (end 138.585 80.038) (width 0.3) (layer "F.Cu") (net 3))
 (segment (start 138.585 80.038) (end 138.585 87.63) (width 0.3) (layer "F.Cu") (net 3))
 (segment (start 128.143 77.724) (end 128.143 81.788) (width 0.4) (layer "F.Cu") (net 1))
 (segment (start 147.0341 83.4144) (end 147.0341 81.1319) (width 0.4) (layer "F.Cu") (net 1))
 (segment (start 149.7326 77.1977) (end 148.9507 76.4158) (width 0.4) (layer "F.Cu") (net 1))
 (segment (start 133.6078 87.2528) (end 137.2078 87.2528) (width 0.4) (layer "F.Cu") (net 1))
 (segment (start 149.7326 78.4334) (end 149.7326 77.1977) (width 0.4) (layer "F.Cu") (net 1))
 (segment (start 137.4373 87.4823) (end 137.585 87.63) (width 0.2998) (layer "F.Cu") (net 1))
 (segment (start 143.085 87.3635) (end 143.085 87.63) (width 0.2998) (layer "F.Cu") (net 1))
 (segment (start 128.143 81.788) (end 133.6078 87.2528) (width 0.4) (layer "F.Cu") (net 1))
 (segment (start 143.2327 87.2158) (end 147.0341 83.4144) (width 0.4) (layer "F.Cu") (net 1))
 (segment (start 143.2327 87.2158) (end 143.085 87.3635) (width 0.2998) (layer "F.Cu") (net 1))
 (segment (start 147.0341 81.1319) (end 149.7326 78.4334) (width 0.4) (layer "F.Cu") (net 1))
 (segment (start 137.2078 87.2528) (end 137.4373 87.4823) (width 0.4) (layer "F.Cu") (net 1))
 (segment (start 148.9507 76.4158) (end 129.4512 76.4158) (width 0.4) (layer "F.Cu") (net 1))
 (segment (start 129.4512 76.4158) (end 128.143 77.724) (width 0.4) (layer "F.Cu") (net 1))
 (segment (start 143.854 91.6741) (end 145.6821 89.846) (width 0.4) (layer "B.Cu") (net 1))
 (segment (start 142.9811 87.7663) (end 142.9811 88.6861) (width 0.4) (layer "B.Cu") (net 1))
 (segment (start 140.8442 80.4841) (end 131.6422 80.4841) (width 0.4) (layer "B.Cu") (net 1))
 (segment (start 141.6173 81.2572) (end 140.8442 80.4841) (width 0.4) (layer "B.Cu") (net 1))
 (segment (start 144.3314 87.2178) (end 143.5296 87.2178) (width 0.4) (layer "B.Cu") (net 1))
 (segment (start 145.6821 89.846) (end 145.6821 88.5685) (width 0.4) (layer "B.Cu") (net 1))
 (segment (start 143.5296 87.2178) (end 142.9811 87.7663) (width 0.4) (layer "B.Cu") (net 1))
 (segment (start 131.6422 80.4841) (end 130.8916 81.2347) (width 0.4) (layer "B.Cu") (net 1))
 (segment (start 137.6619 88.7131) (end 137.6619 87.7579) (width 0.4) (layer "B.Cu") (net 1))
 (segment (start 137.6619 87.7579) (end 141.6173 83.8025) (width 0.4) (layer "B.Cu") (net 1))
 (segment (start 145.6821 88.5685) (end 144.3314 87.2178) (width 0.4) (layer "B.Cu") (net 1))
 (segment (start 141.6173 83.8025) (end 141.6173 81.2572) (width 0.4) (layer "B.Cu") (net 1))
 (segment (start 137.535 88.84) (end 137.6619 88.7131) (width 0.4) (layer "B.Cu") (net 1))
 (segment (start 134.9409 91.6741) (end 143.854 91.6741) (width 0.4) (layer "B.Cu") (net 1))
 (segment (start 130.8916 87.6248) (end 134.9409 91.6741) (width 0.4) (layer "B.Cu") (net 1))
 (segment (start 130.8916 81.2347) (end 130.8916 81.788) (width 0.4) (layer "B.Cu") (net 1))
 (segment (start 130.8916 81.788) (end 130.8916 87.6248) (width 0.4) (layer "B.Cu") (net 1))
 (segment (start 128.143 81.788) (end 130.8916 81.788) (width 0.4) (layer "B.Cu") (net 1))
 (segment (start 142.9811 88.6861) (end 143.135 88.84) (width 0.4) (layer "B.Cu") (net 1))
 (segment (start 141.085 87.63) (end 141.085 86.8281) (width 0.3) (layer "F.Cu") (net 8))
 (segment (start 140.335 77.724) (end 139.0848 78.9742) (width 0.3) (layer "F.Cu") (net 8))
 (segment (start 139.0848 78.9742) (end 139.0848 84.8279) (width 0.3) (layer "F.Cu") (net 8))
 (segment (start 139.0848 84.8279) (end 141.085 86.8281) (width 0.3) (layer "F.Cu") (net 8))
 (segment (start 142.085 87.63) (end 142.085 80.038) (width 0.3) (layer "F.Cu") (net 9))
 (segment (start 142.085 80.038) (end 144.399 77.724) (width 0.3) (layer "F.Cu") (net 9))
 (segment (start 146.4297 79.7573) (end 146.4297 82.9834) (width 0.3) (layer "F.Cu") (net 10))
 (segment (start 146.4297 82.9834) (end 142.585 86.8281) (width 0.3) (layer "F.Cu") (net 10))
 (segment (start 142.585 87.63) (end 142.585 86.8281) (width 0.3) (layer "F.Cu") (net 10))
 (segment (start 148.463 77.724) (end 146.4297 79.7573) (width 0.3) (layer "F.Cu") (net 10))
 (segment (start 135.1487 91.1722) (end 141.24 91.1722) (width 0.3) (layer "B.Cu") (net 11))
 (segment (start 132.207 81.788) (end 132.207 88.2305) (width 0.3) (layer "B.Cu") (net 11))
 (segment (start 141.24 91.1722) (end 142.735 89.6772) (width 0.3) (layer "B.Cu") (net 11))
 (segment (start 132.207 88.2305) (end 135.1487 91.1722) (width 0.3) (layer "B.Cu") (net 11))
 (segment (start 142.735 89.6772) (end 142.735 89.54) (width 0.3) (layer "B.Cu") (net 11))
 (segment (start 136.271 81.788) (end 134.5879 83.4711) (width 0.3) (layer "B.Cu") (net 12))
 (segment (start 134.5879 83.4711) (end 134.5879 89.9724) (width 0.3) (layer "B.Cu") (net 12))
 (segment (start 141.935 89.6704) (end 141.935 89.54) (width 0.3) (layer "B.Cu") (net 12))
 (segment (start 135.3358 90.7203) (end 140.8851 90.7203) (width 0.3) (layer "B.Cu") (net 12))
 (segment (start 140.8851 90.7203) (end 141.935 89.6704) (width 0.3) (layer "B.Cu") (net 12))
 (segment (start 134.5879 89.9724) (end 135.3358 90.7203) (width 0.3) (layer "B.Cu") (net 12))
 (segment (start 139.535 89.6737) (end 138.9527 90.256) (width 0.3) (layer "B.Cu") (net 16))
 (segment (start 135.0515 87.0715) (end 140.335 81.788) (width 0.3) (layer "B.Cu") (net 16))
 (segment (start 139.535 89.54) (end 139.535 89.6737) (width 0.3) (layer "B.Cu") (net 16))
 (segment (start 138.9527 90.256) (end 135.5237 90.256) (width 0.3) (layer "B.Cu") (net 16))
 (segment (start 135.5237 90.256) (end 135.0515 89.7838) (width 0.3) (layer "B.Cu") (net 16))
 (segment (start 135.0515 89.7838) (end 135.0515 87.0715) (width 0.3) (layer "B.Cu") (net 16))
 (segment (start 138.735 89.6027) (end 138.735 89.54) (width 0.3) (layer "F.Cu") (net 17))
 (segment (start 145.1764 90.2527) (end 139.385 90.2527) (width 0.3) (layer "F.Cu") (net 17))
 (segment (start 148.463 81.788) (end 148.463 86.9661) (width 0.3) (layer "F.Cu") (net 17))
 (segment (start 148.463 86.9661) (end 145.1764 90.2527) (width 0.3) (layer "F.Cu") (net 17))
 (segment (start 139.385 90.2527) (end 138.735 89.6027) (width 0.3) (layer "F.Cu") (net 17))
 (segment (start 137.935 89.54) (end 137.935 89.3901) (width 0.3) (layer "B.Cu") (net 18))
 (segment (start 138.4958 88.8293) (end 138.4958 87.6912) (width 0.3) (layer "B.Cu") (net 18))
 (segment (start 137.935 89.3901) (end 138.4958 88.8293) (width 0.3) (layer "B.Cu") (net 18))
 (segment (start 138.4958 87.6912) (end 144.399 81.788) (width 0.3) (layer "B.Cu") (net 18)))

